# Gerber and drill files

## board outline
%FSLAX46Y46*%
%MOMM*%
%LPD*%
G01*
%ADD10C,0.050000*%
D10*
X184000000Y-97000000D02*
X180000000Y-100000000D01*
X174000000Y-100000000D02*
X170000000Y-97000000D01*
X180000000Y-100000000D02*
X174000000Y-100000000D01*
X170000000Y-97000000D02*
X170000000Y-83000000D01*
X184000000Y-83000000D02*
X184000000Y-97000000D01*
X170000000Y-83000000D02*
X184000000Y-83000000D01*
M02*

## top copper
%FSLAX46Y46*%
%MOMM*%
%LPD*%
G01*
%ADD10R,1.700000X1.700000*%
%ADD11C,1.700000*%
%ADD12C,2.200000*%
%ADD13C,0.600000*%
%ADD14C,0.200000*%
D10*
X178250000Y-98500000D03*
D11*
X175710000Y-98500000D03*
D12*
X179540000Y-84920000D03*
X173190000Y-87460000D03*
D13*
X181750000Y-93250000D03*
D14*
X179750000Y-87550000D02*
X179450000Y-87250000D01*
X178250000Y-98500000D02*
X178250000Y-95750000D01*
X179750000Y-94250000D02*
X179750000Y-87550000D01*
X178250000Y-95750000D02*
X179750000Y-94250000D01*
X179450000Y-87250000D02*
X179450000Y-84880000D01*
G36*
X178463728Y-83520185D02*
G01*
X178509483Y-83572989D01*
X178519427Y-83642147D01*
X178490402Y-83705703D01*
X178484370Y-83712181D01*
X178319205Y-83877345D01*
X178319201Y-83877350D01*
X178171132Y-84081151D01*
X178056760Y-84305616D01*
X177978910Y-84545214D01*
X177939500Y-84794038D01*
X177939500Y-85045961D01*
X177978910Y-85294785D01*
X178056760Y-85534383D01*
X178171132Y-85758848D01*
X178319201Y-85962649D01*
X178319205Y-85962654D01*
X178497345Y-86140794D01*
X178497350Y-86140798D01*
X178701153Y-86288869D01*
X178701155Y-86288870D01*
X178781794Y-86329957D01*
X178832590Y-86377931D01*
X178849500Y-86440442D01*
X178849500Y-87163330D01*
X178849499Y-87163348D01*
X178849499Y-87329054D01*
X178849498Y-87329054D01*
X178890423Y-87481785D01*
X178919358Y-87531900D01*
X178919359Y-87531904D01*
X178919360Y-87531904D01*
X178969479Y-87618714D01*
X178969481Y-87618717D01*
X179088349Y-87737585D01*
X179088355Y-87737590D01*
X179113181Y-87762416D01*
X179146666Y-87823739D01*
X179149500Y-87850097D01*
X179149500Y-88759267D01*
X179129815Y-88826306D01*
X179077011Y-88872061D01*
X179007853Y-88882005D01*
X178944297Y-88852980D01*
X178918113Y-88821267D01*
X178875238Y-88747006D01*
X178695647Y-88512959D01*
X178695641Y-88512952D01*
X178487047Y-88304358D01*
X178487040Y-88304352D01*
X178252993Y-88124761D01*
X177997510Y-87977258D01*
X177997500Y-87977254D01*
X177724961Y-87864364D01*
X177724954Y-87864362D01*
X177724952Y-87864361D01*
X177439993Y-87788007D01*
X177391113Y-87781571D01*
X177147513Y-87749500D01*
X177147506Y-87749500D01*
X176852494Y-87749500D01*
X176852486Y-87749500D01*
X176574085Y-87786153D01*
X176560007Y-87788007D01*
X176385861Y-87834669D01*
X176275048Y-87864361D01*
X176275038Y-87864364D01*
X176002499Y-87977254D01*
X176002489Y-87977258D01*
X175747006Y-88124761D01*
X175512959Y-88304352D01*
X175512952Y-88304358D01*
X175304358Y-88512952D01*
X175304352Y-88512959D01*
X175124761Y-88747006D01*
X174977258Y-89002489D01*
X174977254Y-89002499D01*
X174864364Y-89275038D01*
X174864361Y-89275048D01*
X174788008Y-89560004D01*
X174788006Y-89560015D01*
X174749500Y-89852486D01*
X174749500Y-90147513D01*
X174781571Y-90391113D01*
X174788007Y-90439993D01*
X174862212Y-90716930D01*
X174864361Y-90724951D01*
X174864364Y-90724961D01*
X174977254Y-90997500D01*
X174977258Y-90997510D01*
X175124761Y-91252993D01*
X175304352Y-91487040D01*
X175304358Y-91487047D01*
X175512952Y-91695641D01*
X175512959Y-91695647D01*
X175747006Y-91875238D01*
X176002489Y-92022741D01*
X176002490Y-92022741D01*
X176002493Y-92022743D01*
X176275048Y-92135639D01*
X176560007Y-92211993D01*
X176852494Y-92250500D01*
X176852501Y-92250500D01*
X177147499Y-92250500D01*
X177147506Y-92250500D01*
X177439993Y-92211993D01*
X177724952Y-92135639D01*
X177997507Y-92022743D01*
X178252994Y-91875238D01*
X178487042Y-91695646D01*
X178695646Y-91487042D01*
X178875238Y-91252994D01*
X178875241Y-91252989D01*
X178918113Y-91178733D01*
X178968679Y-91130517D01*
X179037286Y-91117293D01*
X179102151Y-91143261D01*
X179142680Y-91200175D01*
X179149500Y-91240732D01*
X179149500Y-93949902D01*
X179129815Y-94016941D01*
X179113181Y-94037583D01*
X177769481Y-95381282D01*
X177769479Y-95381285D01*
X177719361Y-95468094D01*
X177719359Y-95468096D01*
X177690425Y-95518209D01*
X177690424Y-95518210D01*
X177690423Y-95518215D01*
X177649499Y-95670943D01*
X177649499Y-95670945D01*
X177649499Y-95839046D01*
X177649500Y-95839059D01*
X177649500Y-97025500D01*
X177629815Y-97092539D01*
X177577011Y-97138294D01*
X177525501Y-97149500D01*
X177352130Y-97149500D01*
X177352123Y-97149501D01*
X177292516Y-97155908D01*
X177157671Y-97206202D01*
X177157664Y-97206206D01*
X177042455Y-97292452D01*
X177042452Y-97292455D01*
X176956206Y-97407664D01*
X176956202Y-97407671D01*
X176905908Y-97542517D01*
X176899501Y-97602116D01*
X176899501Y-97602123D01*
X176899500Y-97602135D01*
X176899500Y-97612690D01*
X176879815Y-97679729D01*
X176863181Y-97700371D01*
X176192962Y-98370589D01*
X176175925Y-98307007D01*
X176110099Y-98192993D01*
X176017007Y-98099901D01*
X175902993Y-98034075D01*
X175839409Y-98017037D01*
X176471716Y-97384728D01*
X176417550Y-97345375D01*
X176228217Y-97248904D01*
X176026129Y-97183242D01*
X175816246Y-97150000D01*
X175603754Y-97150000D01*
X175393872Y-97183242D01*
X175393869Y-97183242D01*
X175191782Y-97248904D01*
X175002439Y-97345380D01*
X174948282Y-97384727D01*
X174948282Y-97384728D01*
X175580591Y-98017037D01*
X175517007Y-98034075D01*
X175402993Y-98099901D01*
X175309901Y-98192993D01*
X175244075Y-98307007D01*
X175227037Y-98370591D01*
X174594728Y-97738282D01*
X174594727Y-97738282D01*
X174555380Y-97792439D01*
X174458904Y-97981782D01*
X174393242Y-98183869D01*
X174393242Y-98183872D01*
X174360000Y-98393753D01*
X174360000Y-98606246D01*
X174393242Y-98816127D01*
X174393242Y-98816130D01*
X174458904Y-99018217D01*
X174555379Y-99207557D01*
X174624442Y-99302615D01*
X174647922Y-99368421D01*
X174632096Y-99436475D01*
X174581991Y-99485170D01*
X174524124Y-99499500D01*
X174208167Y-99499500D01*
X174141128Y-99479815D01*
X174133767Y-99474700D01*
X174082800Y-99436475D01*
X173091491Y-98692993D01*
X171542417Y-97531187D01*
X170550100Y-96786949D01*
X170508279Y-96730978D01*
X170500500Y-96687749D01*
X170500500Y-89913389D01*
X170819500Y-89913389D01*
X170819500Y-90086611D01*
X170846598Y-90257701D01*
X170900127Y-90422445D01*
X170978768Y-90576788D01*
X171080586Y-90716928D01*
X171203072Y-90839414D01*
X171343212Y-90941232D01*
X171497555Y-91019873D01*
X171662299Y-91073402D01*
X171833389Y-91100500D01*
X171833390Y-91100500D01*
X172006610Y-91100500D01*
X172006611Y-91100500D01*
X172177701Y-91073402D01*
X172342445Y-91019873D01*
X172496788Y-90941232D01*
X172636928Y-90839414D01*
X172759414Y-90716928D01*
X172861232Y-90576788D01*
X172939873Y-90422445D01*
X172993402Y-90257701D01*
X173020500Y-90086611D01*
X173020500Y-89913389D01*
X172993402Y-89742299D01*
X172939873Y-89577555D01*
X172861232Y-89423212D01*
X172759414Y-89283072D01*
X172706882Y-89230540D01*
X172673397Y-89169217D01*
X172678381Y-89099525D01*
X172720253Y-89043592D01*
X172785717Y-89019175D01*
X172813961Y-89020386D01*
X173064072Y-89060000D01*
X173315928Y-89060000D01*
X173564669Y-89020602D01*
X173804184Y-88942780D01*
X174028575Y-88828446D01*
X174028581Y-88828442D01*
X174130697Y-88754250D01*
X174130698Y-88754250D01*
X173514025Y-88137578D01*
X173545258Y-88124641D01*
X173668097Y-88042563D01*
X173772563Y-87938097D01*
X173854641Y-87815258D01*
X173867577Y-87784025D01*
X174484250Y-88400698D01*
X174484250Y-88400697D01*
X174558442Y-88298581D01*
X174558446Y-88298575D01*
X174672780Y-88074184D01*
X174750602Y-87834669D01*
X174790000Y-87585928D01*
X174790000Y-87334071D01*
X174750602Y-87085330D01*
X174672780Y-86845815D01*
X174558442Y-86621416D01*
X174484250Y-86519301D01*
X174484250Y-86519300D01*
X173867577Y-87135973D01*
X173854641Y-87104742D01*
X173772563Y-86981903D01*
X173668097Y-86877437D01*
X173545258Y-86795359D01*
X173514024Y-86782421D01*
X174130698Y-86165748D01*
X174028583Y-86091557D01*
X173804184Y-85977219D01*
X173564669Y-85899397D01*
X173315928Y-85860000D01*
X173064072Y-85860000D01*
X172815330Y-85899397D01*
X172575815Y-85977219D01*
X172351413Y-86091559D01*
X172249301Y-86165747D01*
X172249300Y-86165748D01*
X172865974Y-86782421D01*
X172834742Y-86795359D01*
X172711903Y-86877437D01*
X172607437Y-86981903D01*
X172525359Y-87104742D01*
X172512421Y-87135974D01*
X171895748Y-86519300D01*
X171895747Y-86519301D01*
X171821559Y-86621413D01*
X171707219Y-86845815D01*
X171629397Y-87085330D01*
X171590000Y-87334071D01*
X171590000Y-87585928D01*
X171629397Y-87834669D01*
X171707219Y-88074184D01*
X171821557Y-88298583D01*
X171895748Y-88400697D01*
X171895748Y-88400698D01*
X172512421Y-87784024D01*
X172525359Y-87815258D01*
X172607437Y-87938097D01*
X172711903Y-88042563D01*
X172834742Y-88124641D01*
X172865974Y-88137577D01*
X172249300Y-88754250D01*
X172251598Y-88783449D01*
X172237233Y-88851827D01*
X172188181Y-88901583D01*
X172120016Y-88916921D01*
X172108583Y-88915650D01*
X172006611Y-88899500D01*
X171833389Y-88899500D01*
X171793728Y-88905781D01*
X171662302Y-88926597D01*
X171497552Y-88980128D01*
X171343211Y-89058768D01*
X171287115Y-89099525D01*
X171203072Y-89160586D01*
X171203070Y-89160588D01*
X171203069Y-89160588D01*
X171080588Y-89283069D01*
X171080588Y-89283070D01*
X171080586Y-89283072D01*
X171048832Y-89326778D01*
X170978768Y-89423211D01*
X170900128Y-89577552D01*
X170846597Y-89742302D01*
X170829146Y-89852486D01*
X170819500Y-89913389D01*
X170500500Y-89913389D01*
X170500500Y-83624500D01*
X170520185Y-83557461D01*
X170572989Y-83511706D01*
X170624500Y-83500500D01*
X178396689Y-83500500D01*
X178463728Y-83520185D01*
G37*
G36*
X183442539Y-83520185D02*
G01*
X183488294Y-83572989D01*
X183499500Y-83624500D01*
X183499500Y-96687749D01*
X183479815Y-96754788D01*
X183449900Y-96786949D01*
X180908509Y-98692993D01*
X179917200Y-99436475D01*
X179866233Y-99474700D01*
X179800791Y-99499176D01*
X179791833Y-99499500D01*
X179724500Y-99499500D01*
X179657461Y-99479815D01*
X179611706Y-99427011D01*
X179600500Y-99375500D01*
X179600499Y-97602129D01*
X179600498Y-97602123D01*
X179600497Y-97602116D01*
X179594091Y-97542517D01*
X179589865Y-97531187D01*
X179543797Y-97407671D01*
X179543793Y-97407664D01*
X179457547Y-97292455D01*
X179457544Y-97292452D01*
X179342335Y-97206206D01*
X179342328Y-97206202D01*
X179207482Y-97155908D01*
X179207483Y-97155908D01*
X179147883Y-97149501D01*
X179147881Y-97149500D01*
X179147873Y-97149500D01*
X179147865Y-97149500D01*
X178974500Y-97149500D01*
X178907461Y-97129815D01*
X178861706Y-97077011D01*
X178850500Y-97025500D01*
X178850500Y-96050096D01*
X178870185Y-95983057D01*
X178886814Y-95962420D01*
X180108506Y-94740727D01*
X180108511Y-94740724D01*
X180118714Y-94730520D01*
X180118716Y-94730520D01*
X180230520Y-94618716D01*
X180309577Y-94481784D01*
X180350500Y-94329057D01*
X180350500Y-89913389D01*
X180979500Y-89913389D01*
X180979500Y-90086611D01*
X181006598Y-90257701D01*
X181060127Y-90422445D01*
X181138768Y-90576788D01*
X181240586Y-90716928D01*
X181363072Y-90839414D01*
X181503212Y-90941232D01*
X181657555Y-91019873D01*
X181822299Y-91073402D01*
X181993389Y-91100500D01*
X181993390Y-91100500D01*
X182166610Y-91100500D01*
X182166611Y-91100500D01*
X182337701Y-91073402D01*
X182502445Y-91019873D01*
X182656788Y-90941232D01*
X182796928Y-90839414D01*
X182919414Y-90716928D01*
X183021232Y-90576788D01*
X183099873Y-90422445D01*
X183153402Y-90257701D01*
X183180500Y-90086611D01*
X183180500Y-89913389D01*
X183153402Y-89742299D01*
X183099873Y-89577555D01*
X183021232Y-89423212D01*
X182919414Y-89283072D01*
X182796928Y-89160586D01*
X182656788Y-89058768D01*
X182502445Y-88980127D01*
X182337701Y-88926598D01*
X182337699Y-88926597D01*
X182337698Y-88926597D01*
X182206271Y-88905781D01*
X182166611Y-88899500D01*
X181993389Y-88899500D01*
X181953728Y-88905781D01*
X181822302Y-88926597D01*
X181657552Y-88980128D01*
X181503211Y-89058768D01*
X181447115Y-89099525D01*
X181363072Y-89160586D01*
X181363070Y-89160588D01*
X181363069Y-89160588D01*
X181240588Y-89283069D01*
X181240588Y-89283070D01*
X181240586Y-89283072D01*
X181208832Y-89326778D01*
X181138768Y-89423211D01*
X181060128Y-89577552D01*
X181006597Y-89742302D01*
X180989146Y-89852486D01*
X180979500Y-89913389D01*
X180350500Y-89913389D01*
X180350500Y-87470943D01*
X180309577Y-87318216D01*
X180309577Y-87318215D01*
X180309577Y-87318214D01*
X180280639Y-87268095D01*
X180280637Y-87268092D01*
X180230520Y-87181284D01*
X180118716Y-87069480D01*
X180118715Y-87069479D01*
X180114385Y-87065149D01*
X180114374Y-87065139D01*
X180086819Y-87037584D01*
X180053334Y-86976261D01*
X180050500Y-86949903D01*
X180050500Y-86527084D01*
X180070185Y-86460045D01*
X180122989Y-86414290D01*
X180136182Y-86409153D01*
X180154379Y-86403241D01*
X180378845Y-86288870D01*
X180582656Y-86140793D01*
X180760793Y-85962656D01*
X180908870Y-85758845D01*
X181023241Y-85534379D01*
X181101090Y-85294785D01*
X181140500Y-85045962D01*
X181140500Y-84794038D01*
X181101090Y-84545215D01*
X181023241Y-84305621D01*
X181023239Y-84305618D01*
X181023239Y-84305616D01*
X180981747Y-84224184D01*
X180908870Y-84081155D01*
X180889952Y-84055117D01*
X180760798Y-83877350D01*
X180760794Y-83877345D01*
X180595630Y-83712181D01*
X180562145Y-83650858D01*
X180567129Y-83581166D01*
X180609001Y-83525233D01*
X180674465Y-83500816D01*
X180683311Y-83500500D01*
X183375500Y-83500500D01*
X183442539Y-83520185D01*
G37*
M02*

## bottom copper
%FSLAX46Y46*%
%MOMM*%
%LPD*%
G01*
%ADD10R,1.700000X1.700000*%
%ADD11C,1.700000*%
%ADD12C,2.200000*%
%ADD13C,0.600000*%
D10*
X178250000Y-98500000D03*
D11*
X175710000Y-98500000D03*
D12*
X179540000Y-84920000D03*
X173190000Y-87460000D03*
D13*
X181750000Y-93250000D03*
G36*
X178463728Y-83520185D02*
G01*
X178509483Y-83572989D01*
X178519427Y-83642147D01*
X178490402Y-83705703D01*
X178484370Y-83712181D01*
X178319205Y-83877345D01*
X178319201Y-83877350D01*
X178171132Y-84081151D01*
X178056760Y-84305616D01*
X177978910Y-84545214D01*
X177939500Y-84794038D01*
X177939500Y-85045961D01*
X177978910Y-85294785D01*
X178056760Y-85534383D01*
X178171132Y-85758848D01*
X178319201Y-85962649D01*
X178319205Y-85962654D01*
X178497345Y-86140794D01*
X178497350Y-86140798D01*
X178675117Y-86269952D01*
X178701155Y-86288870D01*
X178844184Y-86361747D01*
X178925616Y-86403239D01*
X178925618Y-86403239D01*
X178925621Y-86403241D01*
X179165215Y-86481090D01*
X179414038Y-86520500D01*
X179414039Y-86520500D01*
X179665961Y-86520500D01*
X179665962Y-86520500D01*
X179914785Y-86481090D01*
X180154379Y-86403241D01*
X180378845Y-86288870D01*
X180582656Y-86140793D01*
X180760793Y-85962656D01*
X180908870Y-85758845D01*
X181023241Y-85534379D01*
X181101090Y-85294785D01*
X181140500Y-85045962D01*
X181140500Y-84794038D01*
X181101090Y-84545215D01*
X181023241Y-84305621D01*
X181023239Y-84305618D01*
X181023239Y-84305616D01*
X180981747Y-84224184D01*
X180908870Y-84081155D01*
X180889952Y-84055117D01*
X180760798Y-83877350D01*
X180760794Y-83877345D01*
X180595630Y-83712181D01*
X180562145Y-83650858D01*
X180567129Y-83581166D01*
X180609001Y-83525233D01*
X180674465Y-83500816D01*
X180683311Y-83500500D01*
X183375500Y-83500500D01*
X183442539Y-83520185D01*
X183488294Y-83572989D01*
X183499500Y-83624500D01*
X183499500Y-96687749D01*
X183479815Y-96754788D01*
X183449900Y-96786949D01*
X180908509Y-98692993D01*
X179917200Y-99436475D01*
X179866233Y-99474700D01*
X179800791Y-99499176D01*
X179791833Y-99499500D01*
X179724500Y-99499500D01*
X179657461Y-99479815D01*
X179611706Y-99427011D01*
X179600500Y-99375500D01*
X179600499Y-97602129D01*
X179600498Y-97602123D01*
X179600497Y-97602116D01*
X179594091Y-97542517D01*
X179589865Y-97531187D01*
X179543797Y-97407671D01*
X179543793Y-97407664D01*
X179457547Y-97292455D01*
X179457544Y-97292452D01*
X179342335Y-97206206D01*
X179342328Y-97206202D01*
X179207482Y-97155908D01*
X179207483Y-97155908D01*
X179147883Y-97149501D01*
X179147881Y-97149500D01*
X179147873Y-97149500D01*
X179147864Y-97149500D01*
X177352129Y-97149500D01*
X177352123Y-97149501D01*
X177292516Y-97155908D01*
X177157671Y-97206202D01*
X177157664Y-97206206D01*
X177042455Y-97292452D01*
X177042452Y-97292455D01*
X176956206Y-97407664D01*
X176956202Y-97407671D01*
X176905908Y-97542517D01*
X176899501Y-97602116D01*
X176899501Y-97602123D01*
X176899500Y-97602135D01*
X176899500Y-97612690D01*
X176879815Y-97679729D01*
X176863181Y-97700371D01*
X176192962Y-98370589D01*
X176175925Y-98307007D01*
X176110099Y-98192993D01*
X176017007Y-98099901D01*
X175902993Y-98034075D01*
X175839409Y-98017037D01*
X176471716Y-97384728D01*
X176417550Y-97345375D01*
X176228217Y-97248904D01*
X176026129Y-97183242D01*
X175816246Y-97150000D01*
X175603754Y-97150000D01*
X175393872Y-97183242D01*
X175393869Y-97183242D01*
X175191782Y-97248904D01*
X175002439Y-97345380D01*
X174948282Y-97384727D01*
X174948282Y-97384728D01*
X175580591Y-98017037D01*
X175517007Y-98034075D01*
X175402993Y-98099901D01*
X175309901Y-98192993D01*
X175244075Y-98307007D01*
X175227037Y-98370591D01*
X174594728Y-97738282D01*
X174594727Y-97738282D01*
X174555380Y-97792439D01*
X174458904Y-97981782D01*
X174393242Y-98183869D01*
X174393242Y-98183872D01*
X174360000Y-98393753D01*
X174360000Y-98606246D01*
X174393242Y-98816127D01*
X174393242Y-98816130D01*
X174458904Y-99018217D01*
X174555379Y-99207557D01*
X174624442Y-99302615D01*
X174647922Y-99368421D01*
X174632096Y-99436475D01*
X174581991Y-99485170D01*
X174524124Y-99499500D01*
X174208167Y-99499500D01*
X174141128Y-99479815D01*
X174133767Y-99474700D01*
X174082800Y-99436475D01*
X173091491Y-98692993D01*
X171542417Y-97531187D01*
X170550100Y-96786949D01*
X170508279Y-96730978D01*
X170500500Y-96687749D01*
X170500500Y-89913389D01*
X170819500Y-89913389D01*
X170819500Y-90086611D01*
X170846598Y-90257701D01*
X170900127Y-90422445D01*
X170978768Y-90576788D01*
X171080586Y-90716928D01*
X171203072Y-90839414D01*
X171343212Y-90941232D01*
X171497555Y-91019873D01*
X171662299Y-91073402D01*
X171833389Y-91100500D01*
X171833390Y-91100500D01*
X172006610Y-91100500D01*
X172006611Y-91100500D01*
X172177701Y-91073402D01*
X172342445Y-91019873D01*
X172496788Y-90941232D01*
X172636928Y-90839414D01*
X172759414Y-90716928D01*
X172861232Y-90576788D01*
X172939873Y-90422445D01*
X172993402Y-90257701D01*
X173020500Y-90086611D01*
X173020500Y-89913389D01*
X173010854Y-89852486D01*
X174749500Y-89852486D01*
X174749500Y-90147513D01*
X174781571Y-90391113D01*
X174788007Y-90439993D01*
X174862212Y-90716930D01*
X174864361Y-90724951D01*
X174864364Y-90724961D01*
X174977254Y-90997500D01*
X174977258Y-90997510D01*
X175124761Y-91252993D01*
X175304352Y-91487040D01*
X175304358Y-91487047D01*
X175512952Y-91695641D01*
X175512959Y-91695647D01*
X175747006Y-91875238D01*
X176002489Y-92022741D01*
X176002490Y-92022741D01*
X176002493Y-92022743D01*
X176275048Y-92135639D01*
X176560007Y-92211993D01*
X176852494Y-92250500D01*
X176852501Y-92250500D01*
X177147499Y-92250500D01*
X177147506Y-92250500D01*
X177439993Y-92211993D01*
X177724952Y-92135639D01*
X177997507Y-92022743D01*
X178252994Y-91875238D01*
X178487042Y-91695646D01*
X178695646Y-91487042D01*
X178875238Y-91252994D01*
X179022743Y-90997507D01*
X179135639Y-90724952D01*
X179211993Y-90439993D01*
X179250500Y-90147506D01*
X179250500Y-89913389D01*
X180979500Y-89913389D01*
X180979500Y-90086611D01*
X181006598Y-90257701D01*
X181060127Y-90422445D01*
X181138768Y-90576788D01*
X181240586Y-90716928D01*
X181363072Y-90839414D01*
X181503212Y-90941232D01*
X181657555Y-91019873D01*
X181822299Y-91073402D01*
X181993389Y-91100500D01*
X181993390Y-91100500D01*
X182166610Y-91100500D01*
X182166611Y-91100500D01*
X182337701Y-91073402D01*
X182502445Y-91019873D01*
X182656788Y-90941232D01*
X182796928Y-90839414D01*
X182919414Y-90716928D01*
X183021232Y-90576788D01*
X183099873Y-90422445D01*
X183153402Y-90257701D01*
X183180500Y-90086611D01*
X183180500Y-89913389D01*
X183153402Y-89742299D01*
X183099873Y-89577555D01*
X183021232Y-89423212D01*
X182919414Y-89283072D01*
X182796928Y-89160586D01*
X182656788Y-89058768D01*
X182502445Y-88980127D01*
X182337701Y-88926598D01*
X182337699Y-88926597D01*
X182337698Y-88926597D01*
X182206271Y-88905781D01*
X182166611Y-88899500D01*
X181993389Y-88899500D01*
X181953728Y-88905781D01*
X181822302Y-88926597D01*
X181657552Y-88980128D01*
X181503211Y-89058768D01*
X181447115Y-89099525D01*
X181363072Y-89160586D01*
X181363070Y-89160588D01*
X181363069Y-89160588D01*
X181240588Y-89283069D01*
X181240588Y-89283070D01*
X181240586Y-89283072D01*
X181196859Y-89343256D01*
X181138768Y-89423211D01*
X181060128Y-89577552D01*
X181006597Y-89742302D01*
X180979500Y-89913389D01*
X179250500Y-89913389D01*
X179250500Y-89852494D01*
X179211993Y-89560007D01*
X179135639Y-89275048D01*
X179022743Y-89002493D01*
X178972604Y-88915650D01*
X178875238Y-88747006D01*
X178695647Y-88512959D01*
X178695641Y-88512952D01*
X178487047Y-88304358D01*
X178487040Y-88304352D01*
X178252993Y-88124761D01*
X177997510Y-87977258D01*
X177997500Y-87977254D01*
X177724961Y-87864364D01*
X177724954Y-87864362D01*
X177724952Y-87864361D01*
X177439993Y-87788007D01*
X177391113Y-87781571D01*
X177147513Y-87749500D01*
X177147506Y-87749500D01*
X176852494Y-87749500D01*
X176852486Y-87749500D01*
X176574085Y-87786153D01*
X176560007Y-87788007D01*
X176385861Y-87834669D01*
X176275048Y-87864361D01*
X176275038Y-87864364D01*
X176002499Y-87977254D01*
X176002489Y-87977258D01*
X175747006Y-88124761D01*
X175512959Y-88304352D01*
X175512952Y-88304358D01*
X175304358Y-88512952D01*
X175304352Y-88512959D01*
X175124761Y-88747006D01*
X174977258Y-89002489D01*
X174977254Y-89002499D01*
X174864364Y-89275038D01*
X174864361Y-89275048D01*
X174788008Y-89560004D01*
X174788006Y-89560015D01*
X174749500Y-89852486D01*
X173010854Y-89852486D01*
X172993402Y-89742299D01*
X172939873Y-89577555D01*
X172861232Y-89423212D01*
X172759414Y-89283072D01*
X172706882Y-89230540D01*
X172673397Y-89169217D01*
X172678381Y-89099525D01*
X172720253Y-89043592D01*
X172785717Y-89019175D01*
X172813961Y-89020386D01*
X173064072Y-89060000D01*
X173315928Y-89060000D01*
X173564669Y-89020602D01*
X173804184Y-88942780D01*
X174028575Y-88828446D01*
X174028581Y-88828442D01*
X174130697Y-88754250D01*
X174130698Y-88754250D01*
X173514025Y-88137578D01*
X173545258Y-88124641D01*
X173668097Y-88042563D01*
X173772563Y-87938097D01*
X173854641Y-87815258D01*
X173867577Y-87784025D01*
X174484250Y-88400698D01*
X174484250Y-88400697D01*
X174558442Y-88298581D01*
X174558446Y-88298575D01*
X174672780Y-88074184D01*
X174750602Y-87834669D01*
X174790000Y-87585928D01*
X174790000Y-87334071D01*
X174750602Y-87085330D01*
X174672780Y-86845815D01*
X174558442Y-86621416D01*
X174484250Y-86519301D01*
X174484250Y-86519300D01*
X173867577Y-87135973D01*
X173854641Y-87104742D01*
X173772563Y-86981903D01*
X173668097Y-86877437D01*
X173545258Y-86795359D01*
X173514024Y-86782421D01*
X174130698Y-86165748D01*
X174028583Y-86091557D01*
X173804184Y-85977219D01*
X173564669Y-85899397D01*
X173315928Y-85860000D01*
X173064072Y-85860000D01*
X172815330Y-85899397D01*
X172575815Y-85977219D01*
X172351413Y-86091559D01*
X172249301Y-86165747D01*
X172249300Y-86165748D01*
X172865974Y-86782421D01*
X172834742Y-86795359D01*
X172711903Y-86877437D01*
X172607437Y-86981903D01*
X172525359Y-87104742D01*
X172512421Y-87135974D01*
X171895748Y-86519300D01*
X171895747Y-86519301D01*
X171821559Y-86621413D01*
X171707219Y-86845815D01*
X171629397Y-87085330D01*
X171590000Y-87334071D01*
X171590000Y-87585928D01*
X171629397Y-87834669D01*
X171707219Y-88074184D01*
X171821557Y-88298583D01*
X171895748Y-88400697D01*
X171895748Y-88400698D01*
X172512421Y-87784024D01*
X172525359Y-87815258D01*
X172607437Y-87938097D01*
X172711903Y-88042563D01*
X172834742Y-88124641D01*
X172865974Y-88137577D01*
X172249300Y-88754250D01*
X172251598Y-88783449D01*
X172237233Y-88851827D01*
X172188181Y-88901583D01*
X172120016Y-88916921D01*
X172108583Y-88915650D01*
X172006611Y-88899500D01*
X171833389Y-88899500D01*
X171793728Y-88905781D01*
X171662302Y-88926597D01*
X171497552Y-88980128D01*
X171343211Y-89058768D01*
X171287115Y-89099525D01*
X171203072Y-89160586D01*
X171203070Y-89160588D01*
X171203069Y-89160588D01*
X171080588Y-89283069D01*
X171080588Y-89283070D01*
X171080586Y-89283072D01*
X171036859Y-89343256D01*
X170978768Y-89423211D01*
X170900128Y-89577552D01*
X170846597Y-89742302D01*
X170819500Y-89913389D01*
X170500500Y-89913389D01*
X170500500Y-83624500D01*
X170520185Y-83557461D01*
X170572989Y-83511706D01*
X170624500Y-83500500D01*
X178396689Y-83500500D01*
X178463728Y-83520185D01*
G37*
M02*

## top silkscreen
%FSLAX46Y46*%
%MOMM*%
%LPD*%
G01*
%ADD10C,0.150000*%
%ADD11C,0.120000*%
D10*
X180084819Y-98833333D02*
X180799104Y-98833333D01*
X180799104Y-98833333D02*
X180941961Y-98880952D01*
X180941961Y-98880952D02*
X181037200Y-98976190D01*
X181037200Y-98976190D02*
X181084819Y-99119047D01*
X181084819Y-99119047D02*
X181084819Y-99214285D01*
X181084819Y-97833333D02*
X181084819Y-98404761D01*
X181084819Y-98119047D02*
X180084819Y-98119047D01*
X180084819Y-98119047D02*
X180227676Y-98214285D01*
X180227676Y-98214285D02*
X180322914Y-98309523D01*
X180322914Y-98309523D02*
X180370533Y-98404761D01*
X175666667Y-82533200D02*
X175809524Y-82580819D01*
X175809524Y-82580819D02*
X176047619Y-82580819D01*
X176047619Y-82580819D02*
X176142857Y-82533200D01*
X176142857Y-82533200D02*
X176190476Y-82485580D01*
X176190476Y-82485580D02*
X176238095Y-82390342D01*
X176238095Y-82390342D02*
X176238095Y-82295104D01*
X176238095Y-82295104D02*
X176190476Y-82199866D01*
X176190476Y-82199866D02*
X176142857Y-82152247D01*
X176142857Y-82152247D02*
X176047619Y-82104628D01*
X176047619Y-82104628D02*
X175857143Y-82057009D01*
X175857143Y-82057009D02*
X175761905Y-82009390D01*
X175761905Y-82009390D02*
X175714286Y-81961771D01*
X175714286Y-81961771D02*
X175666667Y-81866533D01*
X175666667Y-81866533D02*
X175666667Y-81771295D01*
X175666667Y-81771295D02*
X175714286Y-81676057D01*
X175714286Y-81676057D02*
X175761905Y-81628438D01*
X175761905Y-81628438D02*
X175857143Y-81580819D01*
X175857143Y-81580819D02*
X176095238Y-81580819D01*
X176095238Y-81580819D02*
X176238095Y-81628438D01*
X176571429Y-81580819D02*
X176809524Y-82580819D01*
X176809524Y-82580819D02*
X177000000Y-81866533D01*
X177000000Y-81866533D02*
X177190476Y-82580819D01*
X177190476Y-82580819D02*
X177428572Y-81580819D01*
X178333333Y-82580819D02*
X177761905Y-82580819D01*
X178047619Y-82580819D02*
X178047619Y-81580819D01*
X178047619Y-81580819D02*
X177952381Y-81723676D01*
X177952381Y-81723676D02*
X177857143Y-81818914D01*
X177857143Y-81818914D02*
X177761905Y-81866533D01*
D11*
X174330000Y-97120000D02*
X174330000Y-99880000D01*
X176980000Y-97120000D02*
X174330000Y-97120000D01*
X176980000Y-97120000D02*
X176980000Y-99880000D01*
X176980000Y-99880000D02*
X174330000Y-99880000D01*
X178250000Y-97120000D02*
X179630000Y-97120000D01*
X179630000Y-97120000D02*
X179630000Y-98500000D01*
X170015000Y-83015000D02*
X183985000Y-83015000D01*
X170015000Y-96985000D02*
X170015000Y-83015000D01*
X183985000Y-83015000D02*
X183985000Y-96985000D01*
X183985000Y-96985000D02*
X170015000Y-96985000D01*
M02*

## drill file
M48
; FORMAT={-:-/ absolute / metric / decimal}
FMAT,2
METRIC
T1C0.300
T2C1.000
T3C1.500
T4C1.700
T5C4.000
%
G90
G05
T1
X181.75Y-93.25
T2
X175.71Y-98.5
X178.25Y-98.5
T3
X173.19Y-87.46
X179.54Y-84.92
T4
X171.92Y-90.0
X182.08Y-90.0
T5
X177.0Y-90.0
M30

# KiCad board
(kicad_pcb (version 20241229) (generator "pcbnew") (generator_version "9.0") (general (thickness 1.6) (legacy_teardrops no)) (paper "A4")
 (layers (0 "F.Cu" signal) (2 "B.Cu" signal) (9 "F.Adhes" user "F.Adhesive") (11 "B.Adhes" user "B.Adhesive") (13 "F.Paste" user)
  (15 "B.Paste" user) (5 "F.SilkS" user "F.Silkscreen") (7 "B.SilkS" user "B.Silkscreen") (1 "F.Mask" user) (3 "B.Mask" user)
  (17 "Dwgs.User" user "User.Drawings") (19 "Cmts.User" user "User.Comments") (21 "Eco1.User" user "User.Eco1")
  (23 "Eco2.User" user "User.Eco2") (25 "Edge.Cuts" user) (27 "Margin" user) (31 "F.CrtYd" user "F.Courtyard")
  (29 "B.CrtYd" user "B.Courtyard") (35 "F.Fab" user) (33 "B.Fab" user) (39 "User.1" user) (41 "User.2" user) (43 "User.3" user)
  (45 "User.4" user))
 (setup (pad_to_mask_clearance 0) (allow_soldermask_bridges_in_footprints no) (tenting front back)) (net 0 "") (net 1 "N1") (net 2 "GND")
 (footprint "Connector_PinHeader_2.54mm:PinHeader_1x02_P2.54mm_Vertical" (layer "F.Cu") (at 178.25 98.5 -90)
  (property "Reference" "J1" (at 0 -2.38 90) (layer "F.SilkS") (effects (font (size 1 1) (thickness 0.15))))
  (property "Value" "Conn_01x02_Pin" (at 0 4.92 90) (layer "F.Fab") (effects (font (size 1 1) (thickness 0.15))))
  (fp_line (start -1.38 3.92) (end 1.38 3.92) (stroke (width 0.12) (type solid)) (layer "F.SilkS"))
  (fp_line (start -1.38 1.27) (end -1.38 3.92) (stroke (width 0.12) (type solid)) (layer "F.SilkS"))
  (fp_line (start -1.38 1.27) (end 1.38 1.27) (stroke (width 0.12) (type solid)) (layer "F.SilkS"))
  (fp_line (start 1.38 1.27) (end 1.38 3.92) (stroke (width 0.12) (type solid)) (layer "F.SilkS"))
  (fp_line (start -1.38 0) (end -1.38 -1.38) (stroke (width 0.12) (type solid)) (layer "F.SilkS"))
  (fp_line (start -1.38 -1.38) (end 0 -1.38) (stroke (width 0.12) (type solid)) (layer "F.SilkS"))
  (pad "1" thru_hole rect (at 0 0 270) (size 1.7 1.7) (drill 1) (layers "*.Cu" "*.Mask") (remove_unused_layers no) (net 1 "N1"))
  (pad "2" thru_hole circle (at 0 2.54 270) (size 1.7 1.7) (drill 1) (layers "*.Cu" "*.Mask") (remove_unused_layers no) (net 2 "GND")))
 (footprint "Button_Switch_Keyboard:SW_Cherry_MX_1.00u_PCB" (layer "F.Cu") (at 179.54 84.92)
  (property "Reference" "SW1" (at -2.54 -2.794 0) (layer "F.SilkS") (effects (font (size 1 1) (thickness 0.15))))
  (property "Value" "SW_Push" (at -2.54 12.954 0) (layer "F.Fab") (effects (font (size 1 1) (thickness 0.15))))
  (fp_line (start -9.525 -1.905) (end 4.445 -1.905) (stroke (width 0.12) (type solid)) (layer "F.SilkS"))
  (fp_line (start -9.525 12.065) (end -9.525 -1.905) (stroke (width 0.12) (type solid)) (layer "F.SilkS"))
  (fp_line (start 4.445 -1.905) (end 4.445 12.065) (stroke (width 0.12) (type solid)) (layer "F.SilkS"))
  (fp_line (start 4.445 12.065) (end -9.525 12.065) (stroke (width 0.12) (type solid)) (layer "F.SilkS"))
  (pad "" np_thru_hole circle (at -7.62 5.08) (size 1.7 1.7) (drill 1.7) (layers "*.Cu" "*.Mask"))
  (pad "" np_thru_hole circle (at -2.54 5.08) (size 4 4) (drill 4) (layers "*.Cu" "*.Mask"))
  (pad "" np_thru_hole circle (at 2.54 5.08) (size 1.7 1.7) (drill 1.7) (layers "*.Cu" "*.Mask"))
  (pad "1" thru_hole circle (at 0 0) (size 2.2 2.2) (drill 1.5) (layers "*.Cu" "*.Mask") (remove_unused_layers no) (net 1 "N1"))
  (pad "2" thru_hole circle (at -6.35 2.54) (size 2.2 2.2) (drill 1.5) (layers "*.Cu" "*.Mask") (remove_unused_layers no) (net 2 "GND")))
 (gr_line (start 184 97) (end 180 100) (stroke (width 0.05) (type default)) (layer "Edge.Cuts"))
 (gr_line (start 174 100) (end 170 97) (stroke (width 0.05) (type default)) (layer "Edge.Cuts"))
 (gr_line (start 180 100) (end 174 100) (stroke (width 0.05) (type default)) (layer "Edge.Cuts"))
 (gr_line (start 170 97) (end 170 83) (stroke (width 0.05) (type default)) (layer "Edge.Cuts"))
 (gr_line (start 184 83) (end 184 97) (stroke (width 0.05) (type default)) (layer "Edge.Cuts"))
 (gr_line (start 170 83) (end 184 83) (stroke (width 0.05) (type default)) (layer "Edge.Cuts"))
 (via (at 181.75 93.25) (size 0.6) (drill 0.3) (layers "F.Cu" "B.Cu") (free yes) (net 2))
 (segment (start 179.75 87.55) (end 179.45 87.25) (width 0.2) (layer "F.Cu") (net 1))
 (segment (start 178.25 98.5) (end 178.25 95.75) (width 0.2) (layer "F.Cu") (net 1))
 (segment (start 179.75 94.25) (end 179.75 87.55) (width 0.2) (layer "F.Cu") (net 1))
 (segment (start 178.25 95.75) (end 179.75 94.25) (width 0.2) (layer "F.Cu") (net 1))
 (segment (start 179.45 87.25) (end 179.45 84.88) (width 0.2) (layer "F.Cu") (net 1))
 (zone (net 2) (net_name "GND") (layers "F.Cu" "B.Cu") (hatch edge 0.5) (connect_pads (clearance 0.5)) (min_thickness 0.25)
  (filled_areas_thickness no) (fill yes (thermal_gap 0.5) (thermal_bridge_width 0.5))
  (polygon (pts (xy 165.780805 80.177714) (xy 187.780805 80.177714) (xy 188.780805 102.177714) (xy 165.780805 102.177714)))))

